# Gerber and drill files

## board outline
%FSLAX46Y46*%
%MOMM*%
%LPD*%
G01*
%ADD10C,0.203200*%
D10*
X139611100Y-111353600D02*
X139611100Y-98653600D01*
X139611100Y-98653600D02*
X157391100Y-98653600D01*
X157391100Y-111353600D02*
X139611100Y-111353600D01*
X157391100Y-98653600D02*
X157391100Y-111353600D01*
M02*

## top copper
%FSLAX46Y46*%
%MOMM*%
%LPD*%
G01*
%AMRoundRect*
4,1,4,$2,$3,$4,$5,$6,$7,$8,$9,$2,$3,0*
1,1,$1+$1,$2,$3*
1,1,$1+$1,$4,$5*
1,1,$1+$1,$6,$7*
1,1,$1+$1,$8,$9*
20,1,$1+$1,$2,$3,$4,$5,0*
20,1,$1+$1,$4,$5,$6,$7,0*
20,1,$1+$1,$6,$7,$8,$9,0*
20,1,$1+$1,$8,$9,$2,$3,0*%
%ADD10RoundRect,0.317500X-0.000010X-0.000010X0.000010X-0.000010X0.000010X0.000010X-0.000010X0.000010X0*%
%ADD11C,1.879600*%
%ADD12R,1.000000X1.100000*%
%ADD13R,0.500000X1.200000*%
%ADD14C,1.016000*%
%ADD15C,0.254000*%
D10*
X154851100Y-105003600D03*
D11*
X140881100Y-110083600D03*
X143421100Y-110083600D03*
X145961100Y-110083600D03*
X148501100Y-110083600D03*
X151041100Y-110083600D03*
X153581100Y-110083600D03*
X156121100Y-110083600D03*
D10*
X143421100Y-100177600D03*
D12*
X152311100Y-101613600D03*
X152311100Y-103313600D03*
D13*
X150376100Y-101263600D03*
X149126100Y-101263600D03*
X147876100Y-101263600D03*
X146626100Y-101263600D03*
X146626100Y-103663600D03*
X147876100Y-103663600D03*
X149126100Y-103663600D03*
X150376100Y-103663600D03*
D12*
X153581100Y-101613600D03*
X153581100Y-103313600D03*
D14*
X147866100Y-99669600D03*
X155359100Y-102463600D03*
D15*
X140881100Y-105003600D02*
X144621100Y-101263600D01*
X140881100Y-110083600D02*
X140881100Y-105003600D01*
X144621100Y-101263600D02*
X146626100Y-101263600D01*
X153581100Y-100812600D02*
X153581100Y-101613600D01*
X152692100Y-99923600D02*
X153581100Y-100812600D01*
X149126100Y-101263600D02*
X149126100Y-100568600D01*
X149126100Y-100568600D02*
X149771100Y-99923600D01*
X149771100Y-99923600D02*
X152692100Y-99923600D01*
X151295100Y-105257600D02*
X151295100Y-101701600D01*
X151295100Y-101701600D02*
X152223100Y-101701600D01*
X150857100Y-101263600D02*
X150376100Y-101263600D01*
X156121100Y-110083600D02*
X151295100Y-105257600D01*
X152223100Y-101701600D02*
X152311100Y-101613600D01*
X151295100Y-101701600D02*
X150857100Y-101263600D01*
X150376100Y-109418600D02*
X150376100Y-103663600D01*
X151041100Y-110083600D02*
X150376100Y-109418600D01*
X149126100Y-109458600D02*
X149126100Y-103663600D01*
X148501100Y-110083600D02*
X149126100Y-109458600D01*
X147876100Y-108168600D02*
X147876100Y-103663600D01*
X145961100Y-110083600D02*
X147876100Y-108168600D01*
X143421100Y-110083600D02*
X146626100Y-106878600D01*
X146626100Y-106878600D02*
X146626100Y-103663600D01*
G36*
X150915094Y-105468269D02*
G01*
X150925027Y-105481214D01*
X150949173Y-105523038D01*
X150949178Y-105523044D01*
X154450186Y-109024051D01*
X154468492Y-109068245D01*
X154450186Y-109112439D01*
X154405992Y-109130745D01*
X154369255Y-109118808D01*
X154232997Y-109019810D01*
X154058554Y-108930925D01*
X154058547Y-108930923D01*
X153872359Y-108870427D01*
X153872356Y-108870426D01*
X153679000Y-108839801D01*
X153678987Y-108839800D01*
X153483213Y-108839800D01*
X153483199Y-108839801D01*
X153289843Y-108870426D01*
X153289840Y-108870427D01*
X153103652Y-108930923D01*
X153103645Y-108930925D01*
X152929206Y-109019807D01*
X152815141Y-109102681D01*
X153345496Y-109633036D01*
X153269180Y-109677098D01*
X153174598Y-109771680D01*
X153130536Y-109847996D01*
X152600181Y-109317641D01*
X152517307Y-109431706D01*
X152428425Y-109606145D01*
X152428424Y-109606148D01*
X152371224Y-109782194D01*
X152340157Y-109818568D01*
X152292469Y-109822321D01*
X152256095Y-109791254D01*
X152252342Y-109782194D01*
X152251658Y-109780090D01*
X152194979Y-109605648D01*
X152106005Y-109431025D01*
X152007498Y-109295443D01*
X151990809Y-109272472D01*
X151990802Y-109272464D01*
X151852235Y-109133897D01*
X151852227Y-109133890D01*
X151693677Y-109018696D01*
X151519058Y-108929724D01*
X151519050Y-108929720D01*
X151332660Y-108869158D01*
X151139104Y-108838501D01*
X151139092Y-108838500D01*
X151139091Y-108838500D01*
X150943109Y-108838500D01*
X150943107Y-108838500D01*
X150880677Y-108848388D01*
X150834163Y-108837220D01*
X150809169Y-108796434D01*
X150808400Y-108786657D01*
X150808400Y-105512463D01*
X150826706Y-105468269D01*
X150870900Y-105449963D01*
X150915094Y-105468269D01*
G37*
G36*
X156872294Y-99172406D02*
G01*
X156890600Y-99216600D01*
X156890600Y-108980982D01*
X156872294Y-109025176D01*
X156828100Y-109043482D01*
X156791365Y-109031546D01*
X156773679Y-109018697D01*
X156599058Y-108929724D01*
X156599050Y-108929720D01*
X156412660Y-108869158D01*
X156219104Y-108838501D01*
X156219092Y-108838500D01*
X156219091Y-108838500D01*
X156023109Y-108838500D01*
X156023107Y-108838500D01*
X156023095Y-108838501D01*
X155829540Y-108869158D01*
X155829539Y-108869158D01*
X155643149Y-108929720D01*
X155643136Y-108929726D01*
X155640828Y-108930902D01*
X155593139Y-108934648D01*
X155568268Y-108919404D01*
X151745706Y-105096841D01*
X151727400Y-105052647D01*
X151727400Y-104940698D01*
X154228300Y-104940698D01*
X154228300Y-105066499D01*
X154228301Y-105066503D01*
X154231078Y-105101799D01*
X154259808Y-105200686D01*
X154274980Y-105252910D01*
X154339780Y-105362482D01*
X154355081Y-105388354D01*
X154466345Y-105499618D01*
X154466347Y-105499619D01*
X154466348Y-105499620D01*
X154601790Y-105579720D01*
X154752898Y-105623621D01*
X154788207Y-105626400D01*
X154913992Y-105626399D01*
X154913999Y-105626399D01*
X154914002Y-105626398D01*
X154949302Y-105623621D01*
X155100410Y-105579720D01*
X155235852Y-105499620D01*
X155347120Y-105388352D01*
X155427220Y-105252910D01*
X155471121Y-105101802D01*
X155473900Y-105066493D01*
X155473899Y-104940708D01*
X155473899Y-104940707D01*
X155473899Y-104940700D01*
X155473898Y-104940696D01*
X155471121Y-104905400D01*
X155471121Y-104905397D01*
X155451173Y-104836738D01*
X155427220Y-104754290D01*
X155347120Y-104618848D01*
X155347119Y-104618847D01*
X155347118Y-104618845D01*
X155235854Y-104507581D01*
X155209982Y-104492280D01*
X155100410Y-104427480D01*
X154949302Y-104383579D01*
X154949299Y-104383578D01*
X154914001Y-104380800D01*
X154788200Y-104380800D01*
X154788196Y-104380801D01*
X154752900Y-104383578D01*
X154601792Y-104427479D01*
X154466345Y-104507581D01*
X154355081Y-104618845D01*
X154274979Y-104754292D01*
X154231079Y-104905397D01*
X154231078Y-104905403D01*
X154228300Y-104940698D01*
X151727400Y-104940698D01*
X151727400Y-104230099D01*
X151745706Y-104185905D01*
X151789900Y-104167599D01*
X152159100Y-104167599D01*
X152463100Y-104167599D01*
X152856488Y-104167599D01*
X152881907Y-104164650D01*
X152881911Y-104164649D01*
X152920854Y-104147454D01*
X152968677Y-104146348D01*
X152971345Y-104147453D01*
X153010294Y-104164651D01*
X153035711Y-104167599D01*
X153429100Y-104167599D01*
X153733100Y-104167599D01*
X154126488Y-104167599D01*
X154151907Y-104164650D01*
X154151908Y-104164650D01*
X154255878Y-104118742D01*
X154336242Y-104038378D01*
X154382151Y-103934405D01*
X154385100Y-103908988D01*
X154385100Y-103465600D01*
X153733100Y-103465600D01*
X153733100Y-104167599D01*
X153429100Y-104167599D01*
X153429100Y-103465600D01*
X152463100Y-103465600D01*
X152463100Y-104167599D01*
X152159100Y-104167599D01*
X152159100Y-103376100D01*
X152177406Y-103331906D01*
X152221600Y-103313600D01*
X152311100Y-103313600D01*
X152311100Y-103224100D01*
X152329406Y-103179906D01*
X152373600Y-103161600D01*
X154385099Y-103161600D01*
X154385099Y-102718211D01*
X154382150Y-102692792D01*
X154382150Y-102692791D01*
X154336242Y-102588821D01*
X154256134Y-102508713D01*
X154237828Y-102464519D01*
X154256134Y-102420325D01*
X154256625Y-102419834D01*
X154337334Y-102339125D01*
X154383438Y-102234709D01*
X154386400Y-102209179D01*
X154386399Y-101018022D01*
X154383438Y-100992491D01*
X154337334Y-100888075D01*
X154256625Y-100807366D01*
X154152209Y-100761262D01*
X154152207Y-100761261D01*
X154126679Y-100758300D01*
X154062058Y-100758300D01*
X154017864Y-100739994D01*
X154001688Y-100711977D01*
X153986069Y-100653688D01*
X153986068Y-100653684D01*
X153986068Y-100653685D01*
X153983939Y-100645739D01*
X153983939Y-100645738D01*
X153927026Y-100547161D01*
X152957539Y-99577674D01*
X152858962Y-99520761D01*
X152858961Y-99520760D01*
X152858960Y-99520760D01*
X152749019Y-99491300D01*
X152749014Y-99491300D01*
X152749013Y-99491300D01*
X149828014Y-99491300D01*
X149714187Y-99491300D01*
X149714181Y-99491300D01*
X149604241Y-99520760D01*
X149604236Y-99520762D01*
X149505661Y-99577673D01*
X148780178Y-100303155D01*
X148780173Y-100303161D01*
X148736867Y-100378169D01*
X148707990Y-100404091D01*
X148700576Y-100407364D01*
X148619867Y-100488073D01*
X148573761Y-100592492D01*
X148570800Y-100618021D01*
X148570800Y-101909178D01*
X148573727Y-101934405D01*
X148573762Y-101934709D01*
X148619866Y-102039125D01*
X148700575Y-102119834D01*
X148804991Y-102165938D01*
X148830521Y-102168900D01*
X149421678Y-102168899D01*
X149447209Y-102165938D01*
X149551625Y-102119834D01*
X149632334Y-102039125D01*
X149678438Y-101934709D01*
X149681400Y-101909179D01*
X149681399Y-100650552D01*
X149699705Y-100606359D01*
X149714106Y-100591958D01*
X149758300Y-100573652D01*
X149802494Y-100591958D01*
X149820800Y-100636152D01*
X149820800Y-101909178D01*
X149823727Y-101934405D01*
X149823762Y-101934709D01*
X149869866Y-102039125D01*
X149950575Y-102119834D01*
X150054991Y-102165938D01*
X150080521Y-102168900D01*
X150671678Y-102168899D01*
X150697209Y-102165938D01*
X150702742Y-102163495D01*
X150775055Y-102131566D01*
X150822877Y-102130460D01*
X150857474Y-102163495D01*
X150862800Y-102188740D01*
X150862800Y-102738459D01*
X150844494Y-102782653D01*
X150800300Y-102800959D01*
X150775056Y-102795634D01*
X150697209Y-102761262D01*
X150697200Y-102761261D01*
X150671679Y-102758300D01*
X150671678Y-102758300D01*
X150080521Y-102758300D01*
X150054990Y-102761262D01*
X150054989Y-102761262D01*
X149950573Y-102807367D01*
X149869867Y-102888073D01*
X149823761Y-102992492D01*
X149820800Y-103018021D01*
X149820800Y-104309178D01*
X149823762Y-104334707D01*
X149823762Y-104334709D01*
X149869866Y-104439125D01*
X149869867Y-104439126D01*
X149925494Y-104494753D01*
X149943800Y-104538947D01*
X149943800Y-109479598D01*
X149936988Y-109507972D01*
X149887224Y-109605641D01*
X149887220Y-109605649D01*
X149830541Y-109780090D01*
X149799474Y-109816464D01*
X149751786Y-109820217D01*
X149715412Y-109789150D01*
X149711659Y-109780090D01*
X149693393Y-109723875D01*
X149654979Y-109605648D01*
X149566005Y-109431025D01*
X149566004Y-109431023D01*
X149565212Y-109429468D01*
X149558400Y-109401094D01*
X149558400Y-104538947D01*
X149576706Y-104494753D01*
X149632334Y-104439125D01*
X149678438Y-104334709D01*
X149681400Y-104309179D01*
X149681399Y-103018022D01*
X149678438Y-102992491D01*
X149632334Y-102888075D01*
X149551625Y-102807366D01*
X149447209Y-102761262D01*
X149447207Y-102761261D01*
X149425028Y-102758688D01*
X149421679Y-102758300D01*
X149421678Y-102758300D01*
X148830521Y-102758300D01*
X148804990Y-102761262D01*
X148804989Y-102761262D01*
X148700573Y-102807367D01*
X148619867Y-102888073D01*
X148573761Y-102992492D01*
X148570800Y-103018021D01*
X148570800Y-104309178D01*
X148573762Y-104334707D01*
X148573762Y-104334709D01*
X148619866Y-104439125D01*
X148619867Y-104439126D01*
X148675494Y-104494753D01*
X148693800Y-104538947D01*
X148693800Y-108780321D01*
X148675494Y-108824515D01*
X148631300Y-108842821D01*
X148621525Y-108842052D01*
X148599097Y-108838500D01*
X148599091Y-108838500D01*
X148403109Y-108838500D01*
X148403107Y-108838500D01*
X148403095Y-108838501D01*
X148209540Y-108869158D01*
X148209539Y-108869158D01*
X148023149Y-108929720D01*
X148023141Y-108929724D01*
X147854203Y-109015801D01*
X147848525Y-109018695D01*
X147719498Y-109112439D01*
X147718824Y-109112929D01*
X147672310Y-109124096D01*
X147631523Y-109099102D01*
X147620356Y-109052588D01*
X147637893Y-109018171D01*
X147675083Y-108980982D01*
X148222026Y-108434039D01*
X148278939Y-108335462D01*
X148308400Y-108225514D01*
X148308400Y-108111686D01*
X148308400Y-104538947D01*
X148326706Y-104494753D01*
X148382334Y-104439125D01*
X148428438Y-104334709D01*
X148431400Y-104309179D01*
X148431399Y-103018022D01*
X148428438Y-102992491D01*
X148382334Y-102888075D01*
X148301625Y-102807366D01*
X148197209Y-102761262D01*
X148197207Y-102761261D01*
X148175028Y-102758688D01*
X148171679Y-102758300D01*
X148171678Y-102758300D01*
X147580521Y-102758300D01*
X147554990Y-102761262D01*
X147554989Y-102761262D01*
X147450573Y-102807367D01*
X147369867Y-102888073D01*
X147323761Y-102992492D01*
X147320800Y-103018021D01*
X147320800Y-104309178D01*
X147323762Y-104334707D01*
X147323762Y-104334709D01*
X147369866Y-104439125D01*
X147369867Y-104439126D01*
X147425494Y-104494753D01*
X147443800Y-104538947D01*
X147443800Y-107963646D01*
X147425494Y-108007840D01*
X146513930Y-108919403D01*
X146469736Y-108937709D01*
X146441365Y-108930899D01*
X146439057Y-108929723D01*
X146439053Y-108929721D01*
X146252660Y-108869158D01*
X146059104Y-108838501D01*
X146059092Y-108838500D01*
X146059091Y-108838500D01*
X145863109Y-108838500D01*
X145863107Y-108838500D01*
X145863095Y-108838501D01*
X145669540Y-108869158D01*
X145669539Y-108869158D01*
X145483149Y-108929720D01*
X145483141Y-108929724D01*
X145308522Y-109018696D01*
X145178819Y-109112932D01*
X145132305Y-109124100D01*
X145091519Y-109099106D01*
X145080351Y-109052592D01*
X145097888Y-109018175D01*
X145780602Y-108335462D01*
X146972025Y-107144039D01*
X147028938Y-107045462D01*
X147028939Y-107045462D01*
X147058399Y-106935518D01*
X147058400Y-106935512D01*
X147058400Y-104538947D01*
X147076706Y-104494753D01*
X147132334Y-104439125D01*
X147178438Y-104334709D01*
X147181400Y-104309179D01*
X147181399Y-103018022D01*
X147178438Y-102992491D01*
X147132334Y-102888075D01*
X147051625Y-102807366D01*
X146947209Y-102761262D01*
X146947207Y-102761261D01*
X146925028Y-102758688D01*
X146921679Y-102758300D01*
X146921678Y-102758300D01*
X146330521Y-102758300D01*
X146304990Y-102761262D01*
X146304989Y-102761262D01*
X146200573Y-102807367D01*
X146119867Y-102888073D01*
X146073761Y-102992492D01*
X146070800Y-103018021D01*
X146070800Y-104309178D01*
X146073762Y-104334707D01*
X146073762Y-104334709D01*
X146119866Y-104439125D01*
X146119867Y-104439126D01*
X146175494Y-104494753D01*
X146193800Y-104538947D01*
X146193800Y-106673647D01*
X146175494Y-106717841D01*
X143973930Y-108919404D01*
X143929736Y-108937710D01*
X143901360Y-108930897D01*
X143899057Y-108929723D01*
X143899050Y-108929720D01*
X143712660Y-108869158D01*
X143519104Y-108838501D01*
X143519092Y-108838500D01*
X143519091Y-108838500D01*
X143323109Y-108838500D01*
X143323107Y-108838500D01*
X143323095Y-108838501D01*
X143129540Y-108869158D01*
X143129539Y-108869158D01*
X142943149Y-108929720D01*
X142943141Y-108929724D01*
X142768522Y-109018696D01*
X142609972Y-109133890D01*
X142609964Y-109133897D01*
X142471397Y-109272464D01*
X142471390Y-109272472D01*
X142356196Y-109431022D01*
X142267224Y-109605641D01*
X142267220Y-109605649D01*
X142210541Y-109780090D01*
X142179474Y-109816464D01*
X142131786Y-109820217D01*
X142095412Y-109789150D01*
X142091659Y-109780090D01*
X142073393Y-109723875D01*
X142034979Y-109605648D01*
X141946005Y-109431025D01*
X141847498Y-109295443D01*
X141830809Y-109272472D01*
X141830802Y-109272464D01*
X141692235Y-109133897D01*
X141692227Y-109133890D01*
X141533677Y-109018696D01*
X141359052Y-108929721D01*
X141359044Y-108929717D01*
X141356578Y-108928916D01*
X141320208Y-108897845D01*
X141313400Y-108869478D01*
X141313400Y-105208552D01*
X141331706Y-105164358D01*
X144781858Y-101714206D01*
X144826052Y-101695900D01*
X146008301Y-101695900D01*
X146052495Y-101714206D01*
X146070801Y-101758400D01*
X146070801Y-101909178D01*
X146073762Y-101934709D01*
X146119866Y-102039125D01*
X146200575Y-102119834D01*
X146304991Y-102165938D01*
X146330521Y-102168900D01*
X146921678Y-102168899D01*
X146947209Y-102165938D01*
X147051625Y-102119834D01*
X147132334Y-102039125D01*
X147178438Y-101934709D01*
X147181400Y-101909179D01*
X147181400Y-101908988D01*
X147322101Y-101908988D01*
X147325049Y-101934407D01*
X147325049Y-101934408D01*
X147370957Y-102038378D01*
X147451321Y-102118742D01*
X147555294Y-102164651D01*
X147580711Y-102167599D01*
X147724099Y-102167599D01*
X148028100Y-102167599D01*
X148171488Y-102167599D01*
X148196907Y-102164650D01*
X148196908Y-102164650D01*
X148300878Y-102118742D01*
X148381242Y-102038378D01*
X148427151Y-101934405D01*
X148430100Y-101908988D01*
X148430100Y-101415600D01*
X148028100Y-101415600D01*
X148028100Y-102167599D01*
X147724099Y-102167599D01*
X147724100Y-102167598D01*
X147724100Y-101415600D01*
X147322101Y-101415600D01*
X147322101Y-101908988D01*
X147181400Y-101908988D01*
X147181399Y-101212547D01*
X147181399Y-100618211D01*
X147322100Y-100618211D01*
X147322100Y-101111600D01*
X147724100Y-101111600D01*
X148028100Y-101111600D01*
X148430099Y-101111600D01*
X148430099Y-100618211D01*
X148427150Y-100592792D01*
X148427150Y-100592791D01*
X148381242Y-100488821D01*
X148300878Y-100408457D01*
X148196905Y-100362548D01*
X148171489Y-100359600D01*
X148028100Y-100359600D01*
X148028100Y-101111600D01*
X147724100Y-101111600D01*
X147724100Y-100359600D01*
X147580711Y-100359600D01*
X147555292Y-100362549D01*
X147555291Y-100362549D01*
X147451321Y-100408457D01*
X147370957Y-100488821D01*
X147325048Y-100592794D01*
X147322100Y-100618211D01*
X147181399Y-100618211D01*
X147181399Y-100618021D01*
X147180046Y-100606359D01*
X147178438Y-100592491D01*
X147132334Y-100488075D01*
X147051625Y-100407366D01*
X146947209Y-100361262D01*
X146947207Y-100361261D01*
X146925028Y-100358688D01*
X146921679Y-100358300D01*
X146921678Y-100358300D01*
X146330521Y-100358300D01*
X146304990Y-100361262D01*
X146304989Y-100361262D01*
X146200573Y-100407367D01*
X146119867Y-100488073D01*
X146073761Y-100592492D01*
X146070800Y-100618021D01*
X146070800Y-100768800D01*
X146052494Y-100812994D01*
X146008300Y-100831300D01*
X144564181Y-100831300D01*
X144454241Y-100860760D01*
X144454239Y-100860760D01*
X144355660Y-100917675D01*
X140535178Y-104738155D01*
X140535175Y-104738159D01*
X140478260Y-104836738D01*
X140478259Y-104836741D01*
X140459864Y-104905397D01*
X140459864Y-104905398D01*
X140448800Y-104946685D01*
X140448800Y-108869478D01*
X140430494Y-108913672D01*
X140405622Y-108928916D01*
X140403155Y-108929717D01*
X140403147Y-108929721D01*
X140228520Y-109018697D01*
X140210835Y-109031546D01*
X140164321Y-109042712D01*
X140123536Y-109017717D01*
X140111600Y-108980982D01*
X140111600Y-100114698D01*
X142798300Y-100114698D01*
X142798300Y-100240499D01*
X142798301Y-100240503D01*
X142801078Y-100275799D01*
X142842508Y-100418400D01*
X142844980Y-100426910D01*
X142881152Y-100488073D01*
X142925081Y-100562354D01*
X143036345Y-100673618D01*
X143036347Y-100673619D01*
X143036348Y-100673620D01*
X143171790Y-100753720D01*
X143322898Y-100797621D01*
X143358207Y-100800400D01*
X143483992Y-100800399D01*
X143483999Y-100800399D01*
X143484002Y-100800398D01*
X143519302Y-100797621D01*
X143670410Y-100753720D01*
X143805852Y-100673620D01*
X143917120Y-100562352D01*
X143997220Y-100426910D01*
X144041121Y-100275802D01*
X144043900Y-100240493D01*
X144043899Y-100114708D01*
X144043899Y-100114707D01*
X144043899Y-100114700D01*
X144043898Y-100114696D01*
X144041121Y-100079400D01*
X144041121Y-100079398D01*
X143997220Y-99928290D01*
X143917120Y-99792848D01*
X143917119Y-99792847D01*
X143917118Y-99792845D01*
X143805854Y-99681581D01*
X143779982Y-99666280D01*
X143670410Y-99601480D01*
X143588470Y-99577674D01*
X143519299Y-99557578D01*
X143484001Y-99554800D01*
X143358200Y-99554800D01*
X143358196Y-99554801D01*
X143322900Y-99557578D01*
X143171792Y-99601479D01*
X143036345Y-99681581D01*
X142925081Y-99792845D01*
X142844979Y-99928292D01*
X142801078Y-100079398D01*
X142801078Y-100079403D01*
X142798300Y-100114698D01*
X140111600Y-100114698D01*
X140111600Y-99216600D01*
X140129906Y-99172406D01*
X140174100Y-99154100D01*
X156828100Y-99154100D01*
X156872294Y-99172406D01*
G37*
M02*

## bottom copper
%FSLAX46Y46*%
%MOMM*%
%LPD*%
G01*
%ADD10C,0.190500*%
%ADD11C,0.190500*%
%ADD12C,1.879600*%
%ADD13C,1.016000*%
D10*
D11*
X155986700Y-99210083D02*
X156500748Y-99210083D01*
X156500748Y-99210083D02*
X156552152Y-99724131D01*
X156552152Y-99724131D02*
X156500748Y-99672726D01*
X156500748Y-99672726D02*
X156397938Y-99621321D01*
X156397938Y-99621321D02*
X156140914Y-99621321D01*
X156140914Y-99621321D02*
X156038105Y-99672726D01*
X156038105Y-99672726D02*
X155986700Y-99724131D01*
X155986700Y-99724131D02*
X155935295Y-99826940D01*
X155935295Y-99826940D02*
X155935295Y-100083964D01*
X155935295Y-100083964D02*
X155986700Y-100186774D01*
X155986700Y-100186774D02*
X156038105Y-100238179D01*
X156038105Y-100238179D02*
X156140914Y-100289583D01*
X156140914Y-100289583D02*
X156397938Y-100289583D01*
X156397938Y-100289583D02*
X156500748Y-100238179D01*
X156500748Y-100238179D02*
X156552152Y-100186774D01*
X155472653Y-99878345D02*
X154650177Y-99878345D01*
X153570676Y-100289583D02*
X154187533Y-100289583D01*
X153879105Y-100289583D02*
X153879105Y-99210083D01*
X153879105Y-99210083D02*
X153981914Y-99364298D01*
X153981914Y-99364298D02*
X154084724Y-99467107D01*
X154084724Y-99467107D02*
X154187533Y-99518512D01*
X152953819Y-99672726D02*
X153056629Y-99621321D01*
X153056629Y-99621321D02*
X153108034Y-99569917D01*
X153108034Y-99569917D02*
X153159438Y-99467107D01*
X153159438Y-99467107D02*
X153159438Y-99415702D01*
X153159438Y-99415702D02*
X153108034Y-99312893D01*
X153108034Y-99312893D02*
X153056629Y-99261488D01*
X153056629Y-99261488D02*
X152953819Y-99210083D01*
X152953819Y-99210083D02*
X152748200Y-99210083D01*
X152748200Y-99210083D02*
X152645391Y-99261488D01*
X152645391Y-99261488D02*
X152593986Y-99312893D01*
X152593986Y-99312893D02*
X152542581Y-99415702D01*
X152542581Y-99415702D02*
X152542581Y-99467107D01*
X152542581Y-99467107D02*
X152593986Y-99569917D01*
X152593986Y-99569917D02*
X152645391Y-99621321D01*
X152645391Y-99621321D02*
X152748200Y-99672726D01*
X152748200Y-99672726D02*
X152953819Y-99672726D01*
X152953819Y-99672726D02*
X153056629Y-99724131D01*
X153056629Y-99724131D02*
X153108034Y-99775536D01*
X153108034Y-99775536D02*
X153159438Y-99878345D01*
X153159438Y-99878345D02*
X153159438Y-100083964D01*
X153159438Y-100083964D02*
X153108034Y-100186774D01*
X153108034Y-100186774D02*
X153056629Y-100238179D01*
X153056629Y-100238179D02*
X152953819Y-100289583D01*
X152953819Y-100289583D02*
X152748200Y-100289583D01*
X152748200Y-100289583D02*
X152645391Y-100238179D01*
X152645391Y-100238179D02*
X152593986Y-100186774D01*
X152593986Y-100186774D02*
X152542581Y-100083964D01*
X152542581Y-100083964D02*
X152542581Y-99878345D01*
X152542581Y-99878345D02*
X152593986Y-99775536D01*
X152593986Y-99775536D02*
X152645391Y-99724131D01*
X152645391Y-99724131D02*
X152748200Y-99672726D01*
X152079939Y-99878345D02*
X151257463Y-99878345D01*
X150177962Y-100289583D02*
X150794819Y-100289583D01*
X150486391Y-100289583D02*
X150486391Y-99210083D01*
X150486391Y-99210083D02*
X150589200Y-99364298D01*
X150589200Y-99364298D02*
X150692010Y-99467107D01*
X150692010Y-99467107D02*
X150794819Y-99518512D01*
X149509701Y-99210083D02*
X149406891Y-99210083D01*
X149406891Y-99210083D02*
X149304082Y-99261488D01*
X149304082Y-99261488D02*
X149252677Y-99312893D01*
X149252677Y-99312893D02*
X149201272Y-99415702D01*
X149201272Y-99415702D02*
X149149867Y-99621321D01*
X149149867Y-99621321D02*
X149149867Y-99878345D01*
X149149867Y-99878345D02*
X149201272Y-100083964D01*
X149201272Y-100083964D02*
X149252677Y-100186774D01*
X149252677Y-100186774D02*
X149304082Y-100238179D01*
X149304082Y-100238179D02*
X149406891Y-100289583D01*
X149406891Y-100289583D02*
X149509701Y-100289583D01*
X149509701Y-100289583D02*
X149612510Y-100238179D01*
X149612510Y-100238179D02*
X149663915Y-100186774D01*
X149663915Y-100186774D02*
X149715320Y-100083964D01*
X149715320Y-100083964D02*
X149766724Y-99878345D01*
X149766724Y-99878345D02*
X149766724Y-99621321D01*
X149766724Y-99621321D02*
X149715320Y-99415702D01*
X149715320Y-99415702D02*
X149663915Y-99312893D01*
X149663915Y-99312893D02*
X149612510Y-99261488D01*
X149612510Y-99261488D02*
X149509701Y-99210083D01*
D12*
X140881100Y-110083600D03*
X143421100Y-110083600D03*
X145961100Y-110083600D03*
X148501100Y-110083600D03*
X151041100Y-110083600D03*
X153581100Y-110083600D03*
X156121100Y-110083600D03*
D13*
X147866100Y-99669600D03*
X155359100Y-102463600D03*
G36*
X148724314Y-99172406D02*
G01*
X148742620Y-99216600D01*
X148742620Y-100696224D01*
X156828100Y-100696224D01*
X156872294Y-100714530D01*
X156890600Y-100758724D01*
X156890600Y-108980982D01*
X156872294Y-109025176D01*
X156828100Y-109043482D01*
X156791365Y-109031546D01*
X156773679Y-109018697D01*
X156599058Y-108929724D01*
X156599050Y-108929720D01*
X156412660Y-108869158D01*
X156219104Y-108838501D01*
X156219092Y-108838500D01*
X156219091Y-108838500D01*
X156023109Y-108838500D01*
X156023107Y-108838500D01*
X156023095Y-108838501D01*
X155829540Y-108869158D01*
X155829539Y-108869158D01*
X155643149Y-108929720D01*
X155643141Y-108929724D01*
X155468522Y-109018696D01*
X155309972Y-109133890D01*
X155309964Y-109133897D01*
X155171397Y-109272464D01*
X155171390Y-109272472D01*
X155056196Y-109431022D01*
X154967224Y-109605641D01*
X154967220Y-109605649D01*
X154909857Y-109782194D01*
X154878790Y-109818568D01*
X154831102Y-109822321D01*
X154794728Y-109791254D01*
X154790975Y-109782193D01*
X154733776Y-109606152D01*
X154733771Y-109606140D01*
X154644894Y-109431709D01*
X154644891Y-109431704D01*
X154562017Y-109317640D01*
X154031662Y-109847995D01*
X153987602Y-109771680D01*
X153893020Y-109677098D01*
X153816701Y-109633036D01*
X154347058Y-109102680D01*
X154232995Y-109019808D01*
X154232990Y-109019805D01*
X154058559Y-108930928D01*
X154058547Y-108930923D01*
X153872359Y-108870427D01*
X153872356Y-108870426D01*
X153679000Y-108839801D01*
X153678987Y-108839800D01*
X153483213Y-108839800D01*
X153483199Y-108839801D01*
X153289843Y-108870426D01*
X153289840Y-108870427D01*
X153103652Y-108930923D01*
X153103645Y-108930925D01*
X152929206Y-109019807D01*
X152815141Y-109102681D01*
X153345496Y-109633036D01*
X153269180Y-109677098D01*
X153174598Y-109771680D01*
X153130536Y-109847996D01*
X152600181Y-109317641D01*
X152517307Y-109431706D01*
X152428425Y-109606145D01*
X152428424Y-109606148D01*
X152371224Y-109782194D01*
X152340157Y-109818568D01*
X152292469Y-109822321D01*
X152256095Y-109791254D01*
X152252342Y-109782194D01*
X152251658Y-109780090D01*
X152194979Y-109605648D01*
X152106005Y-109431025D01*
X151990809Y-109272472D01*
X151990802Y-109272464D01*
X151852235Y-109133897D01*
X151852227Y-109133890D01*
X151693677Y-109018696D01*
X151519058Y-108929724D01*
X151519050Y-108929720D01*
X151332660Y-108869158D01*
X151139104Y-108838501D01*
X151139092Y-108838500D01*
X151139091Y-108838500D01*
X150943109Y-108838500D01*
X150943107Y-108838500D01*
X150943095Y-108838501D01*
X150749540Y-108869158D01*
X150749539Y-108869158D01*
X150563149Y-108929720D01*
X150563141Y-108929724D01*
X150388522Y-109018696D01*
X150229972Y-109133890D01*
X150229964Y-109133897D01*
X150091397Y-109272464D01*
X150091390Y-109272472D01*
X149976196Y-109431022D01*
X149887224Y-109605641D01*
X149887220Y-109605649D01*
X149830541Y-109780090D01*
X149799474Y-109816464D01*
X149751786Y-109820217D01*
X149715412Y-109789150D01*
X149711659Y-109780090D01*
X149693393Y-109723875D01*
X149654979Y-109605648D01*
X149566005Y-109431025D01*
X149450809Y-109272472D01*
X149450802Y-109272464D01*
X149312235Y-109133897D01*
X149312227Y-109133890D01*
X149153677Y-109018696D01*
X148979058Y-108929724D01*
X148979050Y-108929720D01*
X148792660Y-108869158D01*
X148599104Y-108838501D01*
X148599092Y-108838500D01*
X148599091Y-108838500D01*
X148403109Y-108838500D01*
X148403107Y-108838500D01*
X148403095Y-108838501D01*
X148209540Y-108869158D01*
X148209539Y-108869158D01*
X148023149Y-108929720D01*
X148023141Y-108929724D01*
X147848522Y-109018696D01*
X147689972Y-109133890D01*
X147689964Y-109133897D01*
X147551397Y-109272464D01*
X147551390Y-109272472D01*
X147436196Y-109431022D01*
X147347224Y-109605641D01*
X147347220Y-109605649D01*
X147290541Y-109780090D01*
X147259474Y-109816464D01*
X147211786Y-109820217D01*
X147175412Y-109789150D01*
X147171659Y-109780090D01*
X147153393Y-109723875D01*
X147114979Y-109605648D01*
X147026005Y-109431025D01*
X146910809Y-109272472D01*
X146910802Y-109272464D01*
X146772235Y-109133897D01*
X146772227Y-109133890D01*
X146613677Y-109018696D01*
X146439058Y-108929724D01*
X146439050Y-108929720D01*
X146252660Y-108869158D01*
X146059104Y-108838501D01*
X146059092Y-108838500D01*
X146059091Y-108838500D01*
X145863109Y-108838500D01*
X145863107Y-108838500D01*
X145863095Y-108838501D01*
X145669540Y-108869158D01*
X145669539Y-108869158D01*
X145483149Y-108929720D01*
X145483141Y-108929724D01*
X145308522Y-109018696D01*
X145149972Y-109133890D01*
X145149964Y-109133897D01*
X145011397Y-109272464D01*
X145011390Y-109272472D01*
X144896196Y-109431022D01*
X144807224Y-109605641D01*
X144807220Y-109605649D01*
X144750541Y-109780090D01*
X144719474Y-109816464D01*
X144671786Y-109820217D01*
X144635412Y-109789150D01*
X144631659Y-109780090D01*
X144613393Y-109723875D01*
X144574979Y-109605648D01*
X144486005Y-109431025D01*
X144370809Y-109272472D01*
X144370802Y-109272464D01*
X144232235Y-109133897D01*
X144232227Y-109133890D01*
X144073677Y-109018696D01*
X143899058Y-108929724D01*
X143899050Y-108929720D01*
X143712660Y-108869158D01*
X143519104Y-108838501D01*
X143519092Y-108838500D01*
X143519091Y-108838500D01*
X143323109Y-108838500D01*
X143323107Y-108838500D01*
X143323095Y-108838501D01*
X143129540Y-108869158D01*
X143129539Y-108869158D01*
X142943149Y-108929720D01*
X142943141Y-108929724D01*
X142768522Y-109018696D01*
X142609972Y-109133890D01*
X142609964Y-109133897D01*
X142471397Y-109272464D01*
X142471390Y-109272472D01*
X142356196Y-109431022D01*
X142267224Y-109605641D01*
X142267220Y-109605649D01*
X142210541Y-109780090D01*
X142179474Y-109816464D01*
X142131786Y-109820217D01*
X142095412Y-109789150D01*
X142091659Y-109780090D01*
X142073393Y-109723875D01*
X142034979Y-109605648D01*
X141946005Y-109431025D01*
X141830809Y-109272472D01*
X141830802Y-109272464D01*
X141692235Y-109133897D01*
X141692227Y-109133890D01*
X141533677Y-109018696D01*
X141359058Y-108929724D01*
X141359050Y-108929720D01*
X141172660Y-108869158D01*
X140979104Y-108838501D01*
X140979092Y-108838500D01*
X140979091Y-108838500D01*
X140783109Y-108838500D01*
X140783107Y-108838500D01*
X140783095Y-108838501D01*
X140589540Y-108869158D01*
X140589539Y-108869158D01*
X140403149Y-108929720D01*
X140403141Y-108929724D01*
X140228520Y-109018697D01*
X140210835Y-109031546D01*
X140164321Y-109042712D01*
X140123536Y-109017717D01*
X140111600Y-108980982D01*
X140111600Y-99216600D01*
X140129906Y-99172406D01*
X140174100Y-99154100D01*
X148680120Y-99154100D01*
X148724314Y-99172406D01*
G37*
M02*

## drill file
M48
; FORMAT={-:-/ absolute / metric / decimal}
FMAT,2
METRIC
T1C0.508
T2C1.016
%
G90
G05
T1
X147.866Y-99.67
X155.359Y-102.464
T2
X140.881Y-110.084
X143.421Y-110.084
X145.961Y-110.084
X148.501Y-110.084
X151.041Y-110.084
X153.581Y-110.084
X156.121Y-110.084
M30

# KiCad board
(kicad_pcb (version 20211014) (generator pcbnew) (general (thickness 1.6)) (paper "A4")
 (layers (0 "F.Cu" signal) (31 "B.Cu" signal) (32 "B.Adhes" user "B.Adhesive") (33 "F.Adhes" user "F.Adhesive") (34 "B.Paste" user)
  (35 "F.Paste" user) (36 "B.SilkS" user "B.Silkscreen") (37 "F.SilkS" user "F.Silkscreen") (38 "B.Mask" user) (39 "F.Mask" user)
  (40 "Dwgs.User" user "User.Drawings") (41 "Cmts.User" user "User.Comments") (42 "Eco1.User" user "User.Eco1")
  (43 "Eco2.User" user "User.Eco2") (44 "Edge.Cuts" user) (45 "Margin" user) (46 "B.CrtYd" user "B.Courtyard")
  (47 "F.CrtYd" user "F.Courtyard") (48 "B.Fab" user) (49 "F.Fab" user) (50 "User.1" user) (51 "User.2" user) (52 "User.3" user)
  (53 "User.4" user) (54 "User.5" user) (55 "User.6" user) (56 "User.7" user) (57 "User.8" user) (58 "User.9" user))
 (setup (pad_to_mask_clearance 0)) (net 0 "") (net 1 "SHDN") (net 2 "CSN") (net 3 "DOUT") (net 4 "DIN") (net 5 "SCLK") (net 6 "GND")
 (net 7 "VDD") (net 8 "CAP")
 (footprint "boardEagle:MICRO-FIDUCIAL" (layer "F.Cu") (at 154.8511 105.0036)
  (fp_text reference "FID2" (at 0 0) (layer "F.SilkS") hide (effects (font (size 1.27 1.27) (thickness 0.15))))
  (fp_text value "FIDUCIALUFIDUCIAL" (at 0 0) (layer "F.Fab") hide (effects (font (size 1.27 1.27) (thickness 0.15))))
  (pad "1" smd roundrect (at 0 0) (size 0.635 0.635) (layers "F.Cu" "F.Mask") (roundrect_rratio 0.5) (solder_mask_margin 0.1016)))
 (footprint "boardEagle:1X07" (layer "F.Cu") (at 140.8811 110.0836)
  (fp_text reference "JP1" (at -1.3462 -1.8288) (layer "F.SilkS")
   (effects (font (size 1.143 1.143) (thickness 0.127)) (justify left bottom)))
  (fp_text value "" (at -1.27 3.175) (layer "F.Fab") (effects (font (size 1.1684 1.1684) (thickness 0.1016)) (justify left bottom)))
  (pad "1" thru_hole circle (at 0 0 90) (size 1.8796 1.8796) (drill 1.016) (layers *.Cu *.Mask) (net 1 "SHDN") (solder_mask_margin 0.1016))
  (pad "2" thru_hole circle (at 2.54 0 90) (size 1.8796 1.8796) (drill 1.016) (layers *.Cu *.Mask) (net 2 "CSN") (solder_mask_margin 0.1016))
  (pad "3" thru_hole circle (at 5.08 0 90) (size 1.8796 1.8796) (drill 1.016) (layers *.Cu *.Mask) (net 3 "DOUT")
   (solder_mask_margin 0.1016))
  (pad "4" thru_hole circle (at 7.62 0 90) (size 1.8796 1.8796) (drill 1.016) (layers *.Cu *.Mask) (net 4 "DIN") (solder_mask_margin 0.1016))
  (pad "5" thru_hole circle (at 10.16 0 90) (size 1.8796 1.8796) (drill 1.016) (layers *.Cu *.Mask) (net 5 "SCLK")
   (solder_mask_margin 0.1016))
  (pad "6" thru_hole circle (at 12.7 0 90) (size 1.8796 1.8796) (drill 1.016) (layers *.Cu *.Mask) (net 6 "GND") (solder_mask_margin 0.1016))
  (pad "7" thru_hole circle (at 15.24 0 90) (size 1.8796 1.8796) (drill 1.016) (layers *.Cu *.Mask) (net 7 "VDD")
   (solder_mask_margin 0.1016)))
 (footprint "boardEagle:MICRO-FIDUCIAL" (layer "F.Cu") (at 143.4211 100.1776)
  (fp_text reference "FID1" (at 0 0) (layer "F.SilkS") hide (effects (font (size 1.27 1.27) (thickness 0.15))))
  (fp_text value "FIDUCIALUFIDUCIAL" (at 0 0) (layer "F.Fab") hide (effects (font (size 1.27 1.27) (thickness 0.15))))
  (pad "1" smd roundrect (at 0 0) (size 0.635 0.635) (layers "F.Cu" "F.Mask") (roundrect_rratio 0.5) (solder_mask_margin 0.1016)))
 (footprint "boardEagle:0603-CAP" (layer "F.Cu") (at 152.3111 102.4636 -90)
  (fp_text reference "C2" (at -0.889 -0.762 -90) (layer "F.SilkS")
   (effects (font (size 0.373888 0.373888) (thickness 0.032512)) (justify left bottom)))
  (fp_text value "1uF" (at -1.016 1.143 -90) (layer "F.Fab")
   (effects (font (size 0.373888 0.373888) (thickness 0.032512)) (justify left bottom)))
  (pad "1" smd rect (at -0.85 0 270) (size 1.1 1) (layers "F.Cu" "F.Paste" "F.Mask") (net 7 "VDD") (solder_mask_margin 0.1016))
  (pad "2" smd rect (at 0.85 0 270) (size 1.1 1) (layers "F.Cu" "F.Paste" "F.Mask") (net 6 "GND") (solder_mask_margin 0.1016)))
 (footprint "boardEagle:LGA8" (layer "F.Cu") (at 148.5011 102.4636 -90)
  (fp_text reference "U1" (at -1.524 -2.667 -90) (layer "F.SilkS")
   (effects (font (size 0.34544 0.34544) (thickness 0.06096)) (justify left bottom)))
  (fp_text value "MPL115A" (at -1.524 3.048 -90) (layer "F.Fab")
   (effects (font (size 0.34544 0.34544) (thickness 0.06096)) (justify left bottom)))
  (pad "1" smd rect (at -1.2 -1.875 270) (size 1.2 0.5) (layers "F.Cu" "F.Paste" "F.Mask") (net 7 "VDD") (solder_mask_margin 0.1016))
  (pad "2" smd rect (at -1.2 -0.625 270) (size 1.2 0.5) (layers "F.Cu" "F.Paste" "F.Mask") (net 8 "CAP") (solder_mask_margin 0.1016))
  (pad "3" smd rect (at -1.2 0.625 270) (size 1.2 0.5) (layers "F.Cu" "F.Paste" "F.Mask") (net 6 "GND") (solder_mask_margin 0.1016))
  (pad "4" smd rect (at -1.2 1.875 270) (size 1.2 0.5) (layers "F.Cu" "F.Paste" "F.Mask") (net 1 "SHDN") (solder_mask_margin 0.1016))
  (pad "5" smd rect (at 1.2 1.875 270) (size 1.2 0.5) (layers "F.Cu" "F.Paste" "F.Mask") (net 2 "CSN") (solder_mask_margin 0.1016))
  (pad "6" smd rect (at 1.2 0.625 270) (size 1.2 0.5) (layers "F.Cu" "F.Paste" "F.Mask") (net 3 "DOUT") (solder_mask_margin 0.1016))
  (pad "7" smd rect (at 1.2 -0.625 270) (size 1.2 0.5) (layers "F.Cu" "F.Paste" "F.Mask") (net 4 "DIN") (solder_mask_margin 0.1016))
  (pad "8" smd rect (at 1.2 -1.875 270) (size 1.2 0.5) (layers "F.Cu" "F.Paste" "F.Mask") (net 5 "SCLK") (solder_mask_margin 0.1016)))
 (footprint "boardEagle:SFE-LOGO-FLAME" (layer "F.Cu") (at 140.8811 102.4636)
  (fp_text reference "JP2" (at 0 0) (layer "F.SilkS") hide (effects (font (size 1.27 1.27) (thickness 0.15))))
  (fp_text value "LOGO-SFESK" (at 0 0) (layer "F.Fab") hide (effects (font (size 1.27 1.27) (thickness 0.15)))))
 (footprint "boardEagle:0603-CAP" (layer "F.Cu") (at 153.5811 102.4636 -90)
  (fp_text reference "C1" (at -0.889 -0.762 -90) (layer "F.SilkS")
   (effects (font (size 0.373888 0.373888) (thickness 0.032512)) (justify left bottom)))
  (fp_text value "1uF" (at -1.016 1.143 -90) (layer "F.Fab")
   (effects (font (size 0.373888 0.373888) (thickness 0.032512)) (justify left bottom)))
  (pad "1" smd rect (at -0.85 0 270) (size 1.1 1) (layers "F.Cu" "F.Paste" "F.Mask") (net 8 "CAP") (solder_mask_margin 0.1016))
  (pad "2" smd rect (at 0.85 0 270) (size 1.1 1) (layers "F.Cu" "F.Paste" "F.Mask") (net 6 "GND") (solder_mask_margin 0.1016)))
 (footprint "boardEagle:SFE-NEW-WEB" (layer "B.Cu") (at 154.5971 103.7336 180)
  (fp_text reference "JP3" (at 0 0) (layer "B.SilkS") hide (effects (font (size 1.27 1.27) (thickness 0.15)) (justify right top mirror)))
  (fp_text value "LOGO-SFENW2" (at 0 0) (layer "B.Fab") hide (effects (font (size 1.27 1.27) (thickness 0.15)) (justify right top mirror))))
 (gr_line (start 139.6111 111.3536) (end 139.6111 98.6536) (layer "Edge.Cuts") (width 0.2032))
 (gr_line (start 139.6111 98.6536) (end 157.3911 98.6536) (layer "Edge.Cuts") (width 0.2032))
 (gr_line (start 157.3911 111.3536) (end 139.6111 111.3536) (layer "Edge.Cuts") (width 0.2032))
 (gr_line (start 157.3911 98.6536) (end 157.3911 111.3536) (layer "Edge.Cuts") (width 0.2032))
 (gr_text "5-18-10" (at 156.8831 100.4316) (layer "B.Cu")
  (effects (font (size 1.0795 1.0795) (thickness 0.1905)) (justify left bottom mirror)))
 (segment (start 140.8811 105.0036) (end 144.6211 101.2636) (width 0.254) (layer "F.Cu") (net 1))
 (segment (start 140.8811 110.0836) (end 140.8811 105.0036) (width 0.254) (layer "F.Cu") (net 1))
 (segment (start 144.6211 101.2636) (end 146.6261 101.2636) (width 0.254) (layer "F.Cu") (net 1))
 (via (at 147.8661 99.6696) (size 1.016) (drill 0.508) (layers "F.Cu" "B.Cu") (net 6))
 (via (at 155.3591 102.4636) (size 1.016) (drill 0.508) (layers "F.Cu" "B.Cu") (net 6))
 (segment (start 153.5811 100.8126) (end 153.5811 101.6136) (width 0.254) (layer "F.Cu") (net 8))
 (segment (start 152.6921 99.9236) (end 153.5811 100.8126) (width 0.254) (layer "F.Cu") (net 8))
 (segment (start 149.1261 101.2636) (end 149.1261 100.5686) (width 0.254) (layer "F.Cu") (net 8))
 (segment (start 149.1261 100.5686) (end 149.7711 99.9236) (width 0.254) (layer "F.Cu") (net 8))
 (segment (start 149.7711 99.9236) (end 152.6921 99.9236) (width 0.254) (layer "F.Cu") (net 8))
 (segment (start 151.2951 105.2576) (end 151.2951 101.7016) (width 0.254) (layer "F.Cu") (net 7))
 (segment (start 151.2951 101.7016) (end 152.2231 101.7016) (width 0.254) (layer "F.Cu") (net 7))
 (segment (start 150.8571 101.2636) (end 150.3761 101.2636) (width 0.254) (layer "F.Cu") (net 7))
 (segment (start 156.1211 110.0836) (end 151.2951 105.2576) (width 0.254) (layer "F.Cu") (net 7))
 (segment (start 152.2231 101.7016) (end 152.3111 101.6136) (width 0.254) (layer "F.Cu") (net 7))
 (segment (start 151.2951 101.7016) (end 150.8571 101.2636) (width 0.254) (layer "F.Cu") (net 7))
 (segment (start 150.3761 109.4186) (end 150.3761 103.6636) (width 0.254) (layer "F.Cu") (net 5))
 (segment (start 151.0411 110.0836) (end 150.3761 109.4186) (width 0.254) (layer "F.Cu") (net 5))
 (segment (start 149.1261 109.4586) (end 149.1261 103.6636) (width 0.254) (layer "F.Cu") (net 4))
 (segment (start 148.5011 110.0836) (end 149.1261 109.4586) (width 0.254) (layer "F.Cu") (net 4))
 (segment (start 147.8761 108.1686) (end 147.8761 103.6636) (width 0.254) (layer "F.Cu") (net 3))
 (segment (start 145.9611 110.0836) (end 147.8761 108.1686) (width 0.254) (layer "F.Cu") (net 3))
 (segment (start 143.4211 110.0836) (end 146.6261 106.8786) (width 0.254) (layer "F.Cu") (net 2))
 (segment (start 146.6261 106.8786) (end 146.6261 103.6636) (width 0.254) (layer "F.Cu") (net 2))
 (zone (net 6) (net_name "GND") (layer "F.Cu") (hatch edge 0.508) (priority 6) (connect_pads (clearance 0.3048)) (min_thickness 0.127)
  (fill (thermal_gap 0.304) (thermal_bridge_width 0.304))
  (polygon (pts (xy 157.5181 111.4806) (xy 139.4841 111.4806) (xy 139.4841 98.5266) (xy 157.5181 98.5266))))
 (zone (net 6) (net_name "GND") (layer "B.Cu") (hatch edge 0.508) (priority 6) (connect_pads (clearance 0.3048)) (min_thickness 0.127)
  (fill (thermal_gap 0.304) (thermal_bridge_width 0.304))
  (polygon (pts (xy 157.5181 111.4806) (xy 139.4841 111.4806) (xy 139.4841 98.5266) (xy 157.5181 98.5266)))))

